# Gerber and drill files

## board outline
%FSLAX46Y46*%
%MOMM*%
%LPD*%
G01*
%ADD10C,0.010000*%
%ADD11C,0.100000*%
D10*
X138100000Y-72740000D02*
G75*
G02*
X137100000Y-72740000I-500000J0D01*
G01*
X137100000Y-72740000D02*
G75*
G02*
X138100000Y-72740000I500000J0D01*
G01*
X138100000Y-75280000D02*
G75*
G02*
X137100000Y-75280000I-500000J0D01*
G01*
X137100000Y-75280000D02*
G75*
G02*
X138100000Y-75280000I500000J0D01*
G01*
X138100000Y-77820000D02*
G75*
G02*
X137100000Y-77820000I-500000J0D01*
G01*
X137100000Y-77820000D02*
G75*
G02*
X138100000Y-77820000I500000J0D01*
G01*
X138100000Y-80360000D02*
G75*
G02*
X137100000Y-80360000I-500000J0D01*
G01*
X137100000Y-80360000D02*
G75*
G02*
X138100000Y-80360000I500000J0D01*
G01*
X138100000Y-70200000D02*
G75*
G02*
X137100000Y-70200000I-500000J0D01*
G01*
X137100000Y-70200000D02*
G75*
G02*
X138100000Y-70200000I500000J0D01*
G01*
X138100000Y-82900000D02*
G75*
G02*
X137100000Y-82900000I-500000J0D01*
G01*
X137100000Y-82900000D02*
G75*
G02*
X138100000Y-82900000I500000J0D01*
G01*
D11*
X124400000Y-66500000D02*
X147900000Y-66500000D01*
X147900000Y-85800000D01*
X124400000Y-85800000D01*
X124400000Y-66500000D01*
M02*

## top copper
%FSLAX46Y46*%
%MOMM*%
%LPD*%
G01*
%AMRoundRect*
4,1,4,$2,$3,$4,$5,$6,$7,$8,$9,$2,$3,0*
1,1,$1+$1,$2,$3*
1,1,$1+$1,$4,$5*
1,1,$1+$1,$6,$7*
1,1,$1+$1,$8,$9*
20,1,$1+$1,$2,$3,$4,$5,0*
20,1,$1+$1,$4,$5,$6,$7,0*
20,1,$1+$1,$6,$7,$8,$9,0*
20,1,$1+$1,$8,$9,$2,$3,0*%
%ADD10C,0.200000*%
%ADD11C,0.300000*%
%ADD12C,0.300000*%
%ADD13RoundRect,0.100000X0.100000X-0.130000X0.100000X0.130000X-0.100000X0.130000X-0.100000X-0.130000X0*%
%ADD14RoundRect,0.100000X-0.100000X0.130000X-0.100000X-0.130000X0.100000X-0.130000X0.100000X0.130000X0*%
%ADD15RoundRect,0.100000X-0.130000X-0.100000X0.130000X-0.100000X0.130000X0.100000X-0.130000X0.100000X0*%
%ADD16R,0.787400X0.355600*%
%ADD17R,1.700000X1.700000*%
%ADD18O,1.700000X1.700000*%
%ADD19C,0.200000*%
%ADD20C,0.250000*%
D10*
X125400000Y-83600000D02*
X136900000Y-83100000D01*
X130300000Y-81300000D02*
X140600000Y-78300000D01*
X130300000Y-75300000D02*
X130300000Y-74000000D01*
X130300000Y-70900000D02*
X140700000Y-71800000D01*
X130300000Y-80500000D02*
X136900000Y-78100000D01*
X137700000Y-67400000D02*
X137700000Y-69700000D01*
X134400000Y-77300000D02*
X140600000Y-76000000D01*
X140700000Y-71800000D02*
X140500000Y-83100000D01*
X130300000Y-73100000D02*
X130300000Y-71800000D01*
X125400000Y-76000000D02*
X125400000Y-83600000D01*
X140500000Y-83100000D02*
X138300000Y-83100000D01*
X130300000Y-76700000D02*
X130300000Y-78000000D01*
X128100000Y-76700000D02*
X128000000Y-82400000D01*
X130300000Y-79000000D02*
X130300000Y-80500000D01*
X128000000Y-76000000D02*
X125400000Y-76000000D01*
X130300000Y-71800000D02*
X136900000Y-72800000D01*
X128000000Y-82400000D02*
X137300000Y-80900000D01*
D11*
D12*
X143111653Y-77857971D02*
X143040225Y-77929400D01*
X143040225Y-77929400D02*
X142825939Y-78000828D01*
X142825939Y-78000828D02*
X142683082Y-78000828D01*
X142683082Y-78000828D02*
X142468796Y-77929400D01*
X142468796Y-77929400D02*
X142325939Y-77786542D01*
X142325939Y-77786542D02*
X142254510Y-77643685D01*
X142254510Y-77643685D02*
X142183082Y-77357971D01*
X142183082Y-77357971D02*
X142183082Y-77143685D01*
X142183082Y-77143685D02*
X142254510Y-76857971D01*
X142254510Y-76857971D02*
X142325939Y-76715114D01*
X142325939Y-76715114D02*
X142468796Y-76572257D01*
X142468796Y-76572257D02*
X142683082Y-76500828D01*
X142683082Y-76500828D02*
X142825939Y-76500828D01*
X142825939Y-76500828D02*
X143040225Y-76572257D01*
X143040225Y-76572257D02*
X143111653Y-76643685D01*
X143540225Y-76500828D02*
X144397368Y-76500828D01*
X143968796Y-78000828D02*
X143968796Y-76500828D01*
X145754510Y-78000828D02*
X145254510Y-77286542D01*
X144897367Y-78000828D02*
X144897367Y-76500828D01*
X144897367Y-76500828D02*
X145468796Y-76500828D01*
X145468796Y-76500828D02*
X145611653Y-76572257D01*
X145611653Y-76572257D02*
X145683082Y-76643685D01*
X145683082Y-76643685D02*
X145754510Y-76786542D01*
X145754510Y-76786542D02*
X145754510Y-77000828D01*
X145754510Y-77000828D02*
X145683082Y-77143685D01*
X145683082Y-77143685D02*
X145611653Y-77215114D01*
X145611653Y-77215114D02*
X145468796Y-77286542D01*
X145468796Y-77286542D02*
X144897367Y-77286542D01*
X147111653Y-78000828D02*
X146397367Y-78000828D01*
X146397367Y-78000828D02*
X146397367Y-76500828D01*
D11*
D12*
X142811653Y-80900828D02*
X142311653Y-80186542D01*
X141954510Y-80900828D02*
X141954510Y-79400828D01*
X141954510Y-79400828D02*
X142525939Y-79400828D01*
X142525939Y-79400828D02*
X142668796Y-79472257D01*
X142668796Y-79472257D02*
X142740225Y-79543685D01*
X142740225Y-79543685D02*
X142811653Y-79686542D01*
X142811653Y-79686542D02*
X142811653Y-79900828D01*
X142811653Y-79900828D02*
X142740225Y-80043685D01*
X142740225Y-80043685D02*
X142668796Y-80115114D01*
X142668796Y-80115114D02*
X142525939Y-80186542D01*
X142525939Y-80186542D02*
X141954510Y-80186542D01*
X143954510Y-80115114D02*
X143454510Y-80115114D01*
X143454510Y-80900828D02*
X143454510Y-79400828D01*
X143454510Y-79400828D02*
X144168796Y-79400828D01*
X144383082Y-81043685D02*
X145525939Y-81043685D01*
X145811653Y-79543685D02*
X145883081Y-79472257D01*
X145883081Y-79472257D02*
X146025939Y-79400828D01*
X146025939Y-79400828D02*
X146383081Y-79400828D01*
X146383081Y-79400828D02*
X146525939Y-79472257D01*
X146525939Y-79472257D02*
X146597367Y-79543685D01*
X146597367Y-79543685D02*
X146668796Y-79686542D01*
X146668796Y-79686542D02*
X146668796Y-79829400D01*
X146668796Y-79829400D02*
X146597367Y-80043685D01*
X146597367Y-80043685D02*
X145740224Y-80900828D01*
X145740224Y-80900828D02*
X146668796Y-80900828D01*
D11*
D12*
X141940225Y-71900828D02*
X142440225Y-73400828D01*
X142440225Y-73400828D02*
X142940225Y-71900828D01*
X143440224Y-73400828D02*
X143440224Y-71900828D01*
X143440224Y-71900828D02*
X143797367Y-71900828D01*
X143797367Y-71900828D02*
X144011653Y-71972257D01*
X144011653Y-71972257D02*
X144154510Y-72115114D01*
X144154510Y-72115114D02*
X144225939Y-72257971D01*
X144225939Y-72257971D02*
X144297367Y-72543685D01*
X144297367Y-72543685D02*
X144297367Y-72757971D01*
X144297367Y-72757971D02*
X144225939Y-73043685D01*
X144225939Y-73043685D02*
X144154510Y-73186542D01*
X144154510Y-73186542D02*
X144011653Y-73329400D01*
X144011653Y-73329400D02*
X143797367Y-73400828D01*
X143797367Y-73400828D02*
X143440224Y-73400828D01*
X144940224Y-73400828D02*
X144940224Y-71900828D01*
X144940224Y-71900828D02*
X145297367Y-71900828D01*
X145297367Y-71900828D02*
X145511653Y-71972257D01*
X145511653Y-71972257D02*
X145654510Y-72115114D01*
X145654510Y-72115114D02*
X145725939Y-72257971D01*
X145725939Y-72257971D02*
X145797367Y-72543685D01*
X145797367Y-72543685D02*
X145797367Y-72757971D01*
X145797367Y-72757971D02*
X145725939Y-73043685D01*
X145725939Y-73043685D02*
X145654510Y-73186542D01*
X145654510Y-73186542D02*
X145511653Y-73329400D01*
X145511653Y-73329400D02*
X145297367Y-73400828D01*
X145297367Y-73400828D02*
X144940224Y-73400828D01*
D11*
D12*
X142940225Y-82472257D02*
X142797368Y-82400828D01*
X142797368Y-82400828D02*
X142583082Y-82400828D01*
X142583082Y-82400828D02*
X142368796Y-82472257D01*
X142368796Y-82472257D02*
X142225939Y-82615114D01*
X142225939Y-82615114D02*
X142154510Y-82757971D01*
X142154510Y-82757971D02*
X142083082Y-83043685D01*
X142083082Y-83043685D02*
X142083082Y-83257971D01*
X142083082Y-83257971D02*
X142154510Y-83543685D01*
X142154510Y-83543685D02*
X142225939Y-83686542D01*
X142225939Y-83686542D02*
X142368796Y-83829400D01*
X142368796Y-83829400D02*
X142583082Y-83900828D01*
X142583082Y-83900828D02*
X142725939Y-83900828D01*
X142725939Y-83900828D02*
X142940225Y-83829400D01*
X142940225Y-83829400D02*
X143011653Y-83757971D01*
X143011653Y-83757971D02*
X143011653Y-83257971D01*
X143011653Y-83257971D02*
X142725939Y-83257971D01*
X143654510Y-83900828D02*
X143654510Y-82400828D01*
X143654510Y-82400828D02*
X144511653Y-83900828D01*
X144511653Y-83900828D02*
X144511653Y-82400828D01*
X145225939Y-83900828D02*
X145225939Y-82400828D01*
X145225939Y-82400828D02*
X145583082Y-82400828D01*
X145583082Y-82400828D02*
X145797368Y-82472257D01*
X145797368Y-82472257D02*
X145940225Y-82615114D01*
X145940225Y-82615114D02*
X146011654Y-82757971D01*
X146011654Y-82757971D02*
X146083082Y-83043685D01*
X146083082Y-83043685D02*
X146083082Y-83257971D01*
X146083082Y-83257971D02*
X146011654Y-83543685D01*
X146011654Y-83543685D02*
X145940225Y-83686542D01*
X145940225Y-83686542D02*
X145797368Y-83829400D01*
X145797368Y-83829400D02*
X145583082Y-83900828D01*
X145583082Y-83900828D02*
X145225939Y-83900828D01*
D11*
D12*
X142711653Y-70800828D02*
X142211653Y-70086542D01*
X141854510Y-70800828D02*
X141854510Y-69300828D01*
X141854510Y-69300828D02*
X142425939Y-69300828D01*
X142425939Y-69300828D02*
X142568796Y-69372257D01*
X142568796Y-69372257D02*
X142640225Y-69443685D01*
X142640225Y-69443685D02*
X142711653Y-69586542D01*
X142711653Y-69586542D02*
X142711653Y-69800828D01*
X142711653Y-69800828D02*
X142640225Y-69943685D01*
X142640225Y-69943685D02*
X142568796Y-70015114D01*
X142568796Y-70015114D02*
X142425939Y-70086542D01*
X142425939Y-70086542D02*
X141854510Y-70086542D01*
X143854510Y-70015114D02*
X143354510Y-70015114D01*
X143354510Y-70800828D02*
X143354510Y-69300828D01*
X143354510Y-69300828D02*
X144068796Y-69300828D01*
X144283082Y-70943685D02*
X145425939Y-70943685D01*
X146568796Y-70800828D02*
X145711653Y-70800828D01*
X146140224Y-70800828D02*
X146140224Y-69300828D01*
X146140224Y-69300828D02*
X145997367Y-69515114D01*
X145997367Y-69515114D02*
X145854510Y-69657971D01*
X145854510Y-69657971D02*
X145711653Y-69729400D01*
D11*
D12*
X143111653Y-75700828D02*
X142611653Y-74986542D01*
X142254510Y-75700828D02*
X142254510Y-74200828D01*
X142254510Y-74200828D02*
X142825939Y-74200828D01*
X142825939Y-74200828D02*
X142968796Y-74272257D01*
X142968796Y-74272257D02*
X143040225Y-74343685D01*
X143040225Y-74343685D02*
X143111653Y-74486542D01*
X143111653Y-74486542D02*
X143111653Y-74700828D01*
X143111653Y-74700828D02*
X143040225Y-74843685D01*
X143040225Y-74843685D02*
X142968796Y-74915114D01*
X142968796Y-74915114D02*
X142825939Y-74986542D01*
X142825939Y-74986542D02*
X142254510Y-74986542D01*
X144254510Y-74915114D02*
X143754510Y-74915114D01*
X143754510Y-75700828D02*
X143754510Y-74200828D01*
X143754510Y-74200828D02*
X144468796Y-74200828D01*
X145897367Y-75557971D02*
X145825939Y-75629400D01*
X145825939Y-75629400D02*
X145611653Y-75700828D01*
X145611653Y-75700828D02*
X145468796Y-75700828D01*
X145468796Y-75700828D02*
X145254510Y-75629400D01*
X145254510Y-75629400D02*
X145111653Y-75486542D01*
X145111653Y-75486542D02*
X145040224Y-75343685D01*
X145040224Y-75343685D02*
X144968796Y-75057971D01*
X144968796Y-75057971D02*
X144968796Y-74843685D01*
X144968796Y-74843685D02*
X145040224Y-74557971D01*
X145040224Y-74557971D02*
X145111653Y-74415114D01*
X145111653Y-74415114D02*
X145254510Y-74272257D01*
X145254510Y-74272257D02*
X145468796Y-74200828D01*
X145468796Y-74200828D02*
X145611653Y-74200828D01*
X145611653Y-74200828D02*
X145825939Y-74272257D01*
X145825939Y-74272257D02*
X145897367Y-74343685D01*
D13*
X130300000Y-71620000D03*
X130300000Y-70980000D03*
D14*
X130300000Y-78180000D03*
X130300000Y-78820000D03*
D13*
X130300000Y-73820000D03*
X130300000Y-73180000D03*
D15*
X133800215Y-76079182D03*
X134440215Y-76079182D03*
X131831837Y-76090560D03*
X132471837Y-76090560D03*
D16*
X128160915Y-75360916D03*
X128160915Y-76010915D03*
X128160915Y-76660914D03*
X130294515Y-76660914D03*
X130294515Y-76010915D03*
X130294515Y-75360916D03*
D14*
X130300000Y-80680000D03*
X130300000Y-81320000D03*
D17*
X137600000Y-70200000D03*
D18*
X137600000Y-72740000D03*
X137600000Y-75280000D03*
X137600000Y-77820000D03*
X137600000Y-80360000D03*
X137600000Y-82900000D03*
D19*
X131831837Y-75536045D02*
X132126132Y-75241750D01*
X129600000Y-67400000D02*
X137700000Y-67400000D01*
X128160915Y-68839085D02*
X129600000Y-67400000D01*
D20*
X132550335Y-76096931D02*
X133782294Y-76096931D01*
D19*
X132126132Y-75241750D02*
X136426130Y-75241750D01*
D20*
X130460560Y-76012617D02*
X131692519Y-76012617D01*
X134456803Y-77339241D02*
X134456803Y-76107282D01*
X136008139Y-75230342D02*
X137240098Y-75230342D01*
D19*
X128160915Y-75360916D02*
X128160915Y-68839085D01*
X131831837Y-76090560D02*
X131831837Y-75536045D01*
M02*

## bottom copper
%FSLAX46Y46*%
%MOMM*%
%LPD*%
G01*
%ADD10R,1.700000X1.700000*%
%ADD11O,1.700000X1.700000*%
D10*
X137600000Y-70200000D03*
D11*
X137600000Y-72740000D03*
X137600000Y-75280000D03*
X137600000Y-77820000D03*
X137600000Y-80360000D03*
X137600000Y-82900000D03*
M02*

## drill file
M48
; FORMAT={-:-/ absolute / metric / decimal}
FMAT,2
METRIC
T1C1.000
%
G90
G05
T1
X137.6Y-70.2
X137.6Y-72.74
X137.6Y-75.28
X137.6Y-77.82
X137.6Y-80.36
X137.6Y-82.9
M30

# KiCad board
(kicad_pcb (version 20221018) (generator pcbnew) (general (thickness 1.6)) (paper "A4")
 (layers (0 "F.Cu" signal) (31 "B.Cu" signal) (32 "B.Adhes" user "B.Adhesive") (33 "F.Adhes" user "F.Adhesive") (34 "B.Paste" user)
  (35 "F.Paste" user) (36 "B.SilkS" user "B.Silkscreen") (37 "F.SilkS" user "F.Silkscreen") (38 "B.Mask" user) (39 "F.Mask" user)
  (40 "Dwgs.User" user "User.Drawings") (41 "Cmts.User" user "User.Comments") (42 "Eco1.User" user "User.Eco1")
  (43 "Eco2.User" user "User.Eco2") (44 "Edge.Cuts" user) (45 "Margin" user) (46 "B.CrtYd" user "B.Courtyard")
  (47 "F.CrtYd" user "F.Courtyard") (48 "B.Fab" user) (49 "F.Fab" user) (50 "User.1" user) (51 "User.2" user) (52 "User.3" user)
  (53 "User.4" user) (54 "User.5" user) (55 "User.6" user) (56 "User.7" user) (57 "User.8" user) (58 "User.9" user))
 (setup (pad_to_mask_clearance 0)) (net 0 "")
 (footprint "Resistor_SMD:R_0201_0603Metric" (layer "F.Cu") (at 130.3 71.3 90)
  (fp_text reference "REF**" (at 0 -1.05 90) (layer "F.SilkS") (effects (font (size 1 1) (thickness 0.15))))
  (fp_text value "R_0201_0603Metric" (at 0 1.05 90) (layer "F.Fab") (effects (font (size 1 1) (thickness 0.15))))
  (pad "" smd roundrect (at -0.345 0 90) (size 0.318 0.36) (layers "F.Paste") (roundrect_rratio 0.25))
  (pad "" smd roundrect (at 0.345 0 90) (size 0.318 0.36) (layers "F.Paste") (roundrect_rratio 0.25))
  (pad "1" smd roundrect (at -0.32 0 90) (size 0.46 0.4) (layers "F.Cu" "F.Mask") (roundrect_rratio 0.25))
  (pad "2" smd roundrect (at 0.32 0 90) (size 0.46 0.4) (layers "F.Cu" "F.Mask") (roundrect_rratio 0.25)))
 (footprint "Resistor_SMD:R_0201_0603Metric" (layer "F.Cu") (at 130.3 78.5 -90)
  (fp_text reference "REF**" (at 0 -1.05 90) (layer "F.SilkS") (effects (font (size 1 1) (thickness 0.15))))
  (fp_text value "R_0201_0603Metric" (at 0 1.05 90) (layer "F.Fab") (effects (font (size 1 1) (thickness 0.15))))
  (pad "" smd roundrect (at -0.345 0 270) (size 0.318 0.36) (layers "F.Paste") (roundrect_rratio 0.25))
  (pad "" smd roundrect (at 0.345 0 270) (size 0.318 0.36) (layers "F.Paste") (roundrect_rratio 0.25))
  (pad "1" smd roundrect (at -0.32 0 270) (size 0.46 0.4) (layers "F.Cu" "F.Mask") (roundrect_rratio 0.25))
  (pad "2" smd roundrect (at 0.32 0 270) (size 0.46 0.4) (layers "F.Cu" "F.Mask") (roundrect_rratio 0.25)))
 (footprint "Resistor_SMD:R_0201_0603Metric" (layer "F.Cu") (at 130.3 73.5 90)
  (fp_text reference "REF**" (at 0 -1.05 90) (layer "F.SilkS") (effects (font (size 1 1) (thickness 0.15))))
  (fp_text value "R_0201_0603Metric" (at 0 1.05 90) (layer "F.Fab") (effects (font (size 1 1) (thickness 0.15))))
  (pad "" smd roundrect (at -0.345 0 90) (size 0.318 0.36) (layers "F.Paste") (roundrect_rratio 0.25))
  (pad "" smd roundrect (at 0.345 0 90) (size 0.318 0.36) (layers "F.Paste") (roundrect_rratio 0.25))
  (pad "1" smd roundrect (at -0.32 0 90) (size 0.46 0.4) (layers "F.Cu" "F.Mask") (roundrect_rratio 0.25))
  (pad "2" smd roundrect (at 0.32 0 90) (size 0.46 0.4) (layers "F.Cu" "F.Mask") (roundrect_rratio 0.25)))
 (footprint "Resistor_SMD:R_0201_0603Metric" (layer "F.Cu") (at 134.120215 76.079182)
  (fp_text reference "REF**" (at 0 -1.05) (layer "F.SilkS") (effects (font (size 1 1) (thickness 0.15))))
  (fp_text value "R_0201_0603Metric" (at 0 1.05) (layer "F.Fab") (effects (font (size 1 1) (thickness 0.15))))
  (pad "" smd roundrect (at -0.345 0) (size 0.318 0.36) (layers "F.Paste") (roundrect_rratio 0.25))
  (pad "" smd roundrect (at 0.345 0) (size 0.318 0.36) (layers "F.Paste") (roundrect_rratio 0.25))
  (pad "1" smd roundrect (at -0.32 0) (size 0.46 0.4) (layers "F.Cu" "F.Mask") (roundrect_rratio 0.25))
  (pad "2" smd roundrect (at 0.32 0) (size 0.46 0.4) (layers "F.Cu" "F.Mask") (roundrect_rratio 0.25)))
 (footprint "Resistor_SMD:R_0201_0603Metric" (layer "F.Cu") (at 132.151837 76.09056)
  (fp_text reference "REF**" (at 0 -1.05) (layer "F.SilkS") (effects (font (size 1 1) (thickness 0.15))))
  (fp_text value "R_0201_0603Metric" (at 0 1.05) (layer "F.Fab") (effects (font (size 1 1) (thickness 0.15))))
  (pad "" smd roundrect (at -0.345 0) (size 0.318 0.36) (layers "F.Paste") (roundrect_rratio 0.25))
  (pad "" smd roundrect (at 0.345 0) (size 0.318 0.36) (layers "F.Paste") (roundrect_rratio 0.25))
  (pad "1" smd roundrect (at -0.32 0) (size 0.46 0.4) (layers "F.Cu" "F.Mask") (roundrect_rratio 0.25))
  (pad "2" smd roundrect (at 0.32 0) (size 0.46 0.4) (layers "F.Cu" "F.Mask") (roundrect_rratio 0.25)))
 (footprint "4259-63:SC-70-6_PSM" (layer "F.Cu") (at 129.227715 76.010915)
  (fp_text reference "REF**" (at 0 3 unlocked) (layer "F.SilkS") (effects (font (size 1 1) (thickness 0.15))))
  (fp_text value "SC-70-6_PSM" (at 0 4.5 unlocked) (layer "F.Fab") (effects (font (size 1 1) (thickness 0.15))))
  (pad "1" smd rect (at -1.0668 -0.649999) (size 0.7874 0.3556) (layers "F.Cu" "F.Paste" "F.Mask"))
  (pad "2" smd rect (at -1.0668 0) (size 0.7874 0.3556) (layers "F.Cu" "F.Paste" "F.Mask"))
  (pad "3" smd rect (at -1.0668 0.649999) (size 0.7874 0.3556) (layers "F.Cu" "F.Paste" "F.Mask"))
  (pad "4" smd rect (at 1.0668 0.649999) (size 0.7874 0.3556) (layers "F.Cu" "F.Paste" "F.Mask"))
  (pad "5" smd rect (at 1.0668 0) (size 0.7874 0.3556) (layers "F.Cu" "F.Paste" "F.Mask"))
  (pad "6" smd rect (at 1.0668 -0.649999) (size 0.7874 0.3556) (layers "F.Cu" "F.Paste" "F.Mask")))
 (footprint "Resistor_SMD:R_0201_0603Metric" (layer "F.Cu") (at 130.3 81 -90)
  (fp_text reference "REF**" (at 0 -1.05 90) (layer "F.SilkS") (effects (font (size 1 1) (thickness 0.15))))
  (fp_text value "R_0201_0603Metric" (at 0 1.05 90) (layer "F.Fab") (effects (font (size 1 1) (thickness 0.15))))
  (pad "" smd roundrect (at -0.345 0 270) (size 0.318 0.36) (layers "F.Paste") (roundrect_rratio 0.25))
  (pad "" smd roundrect (at 0.345 0 270) (size 0.318 0.36) (layers "F.Paste") (roundrect_rratio 0.25))
  (pad "1" smd roundrect (at -0.32 0 270) (size 0.46 0.4) (layers "F.Cu" "F.Mask") (roundrect_rratio 0.25))
  (pad "2" smd roundrect (at 0.32 0 270) (size 0.46 0.4) (layers "F.Cu" "F.Mask") (roundrect_rratio 0.25)))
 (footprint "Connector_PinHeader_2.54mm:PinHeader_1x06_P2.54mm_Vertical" (layer "F.Cu") (at 137.6 70.2)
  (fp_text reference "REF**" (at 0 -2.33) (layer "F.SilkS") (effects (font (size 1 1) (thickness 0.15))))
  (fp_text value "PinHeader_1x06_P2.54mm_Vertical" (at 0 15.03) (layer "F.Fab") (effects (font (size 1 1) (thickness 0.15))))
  (pad "1" thru_hole rect (at 0 0) (size 1.7 1.7) (drill 1) (layers "*.Cu" "*.Mask"))
  (pad "2" thru_hole oval (at 0 2.54) (size 1.7 1.7) (drill 1) (layers "*.Cu" "*.Mask"))
  (pad "3" thru_hole oval (at 0 5.08) (size 1.7 1.7) (drill 1) (layers "*.Cu" "*.Mask"))
  (pad "4" thru_hole oval (at 0 7.62) (size 1.7 1.7) (drill 1) (layers "*.Cu" "*.Mask"))
  (pad "5" thru_hole oval (at 0 10.16) (size 1.7 1.7) (drill 1) (layers "*.Cu" "*.Mask"))
  (pad "6" thru_hole oval (at 0 12.7) (size 1.7 1.7) (drill 1) (layers "*.Cu" "*.Mask")))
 (gr_line (start 125.4 83.6) (end 136.9 83.1) (stroke (width 0.2) (type default)) (layer "F.Cu"))
 (gr_line (start 130.3 81.3) (end 140.6 78.3) (stroke (width 0.2) (type default)) (layer "F.Cu"))
 (gr_line (start 130.3 75.3) (end 130.3 74) (stroke (width 0.2) (type default)) (layer "F.Cu"))
 (gr_line (start 130.3 70.9) (end 140.7 71.8) (stroke (width 0.2) (type default)) (layer "F.Cu"))
 (gr_line (start 130.3 80.5) (end 136.9 78.1) (stroke (width 0.2) (type default)) (layer "F.Cu"))
 (gr_line (start 137.7 67.4) (end 137.7 69.7) (stroke (width 0.2) (type default)) (layer "F.Cu"))
 (gr_line (start 134.4 77.3) (end 140.6 76) (stroke (width 0.2) (type default)) (layer "F.Cu"))
 (gr_line (start 140.7 71.8) (end 140.5 83.1) (stroke (width 0.2) (type default)) (layer "F.Cu"))
 (gr_line (start 130.3 73.1) (end 130.3 71.8) (stroke (width 0.2) (type default)) (layer "F.Cu"))
 (gr_line (start 125.4 76) (end 125.4 83.6) (stroke (width 0.2) (type default)) (layer "F.Cu"))
 (gr_line (start 140.5 83.1) (end 138.3 83.1) (stroke (width 0.2) (type default)) (layer "F.Cu"))
 (gr_line (start 130.3 76.7) (end 130.3 78) (stroke (width 0.2) (type default)) (layer "F.Cu"))
 (gr_line (start 128.1 76.7) (end 128 82.4) (stroke (width 0.2) (type default)) (layer "F.Cu"))
 (gr_line (start 130.3 79) (end 130.3 80.5) (stroke (width 0.2) (type default)) (layer "F.Cu"))
 (gr_line (start 128 76) (end 125.4 76) (stroke (width 0.2) (type default)) (layer "F.Cu"))
 (gr_line (start 130.3 71.8) (end 136.9 72.8) (stroke (width 0.2) (type default)) (layer "F.Cu"))
 (gr_line (start 128 82.4) (end 137.3 80.9) (stroke (width 0.2) (type default)) (layer "F.Cu"))
 (gr_circle (center 137.6 72.74) (end 138.1 72.74) (stroke (width 0.01) (type default)) (fill none) (layer "Edge.Cuts"))
 (gr_circle (center 137.6 75.28) (end 138.1 75.28) (stroke (width 0.01) (type default)) (fill none) (layer "Edge.Cuts"))
 (gr_circle (center 137.6 77.82) (end 138.1 77.82) (stroke (width 0.01) (type default)) (fill none) (layer "Edge.Cuts"))
 (gr_circle (center 137.6 80.36) (end 138.1 80.36) (stroke (width 0.01) (type default)) (fill none) (layer "Edge.Cuts"))
 (gr_circle (center 137.6 70.2) (end 138.1 70.2) (stroke (width 0.01) (type default)) (fill none) (layer "Edge.Cuts"))
 (gr_circle (center 137.6 82.9) (end 138.1 82.9) (stroke (width 0.01) (type default)) (fill none) (layer "Edge.Cuts"))
 (gr_rect (start 124.4 66.5) (end 147.9 85.8) (stroke (width 0.1) (type default)) (fill none) (layer "Edge.Cuts"))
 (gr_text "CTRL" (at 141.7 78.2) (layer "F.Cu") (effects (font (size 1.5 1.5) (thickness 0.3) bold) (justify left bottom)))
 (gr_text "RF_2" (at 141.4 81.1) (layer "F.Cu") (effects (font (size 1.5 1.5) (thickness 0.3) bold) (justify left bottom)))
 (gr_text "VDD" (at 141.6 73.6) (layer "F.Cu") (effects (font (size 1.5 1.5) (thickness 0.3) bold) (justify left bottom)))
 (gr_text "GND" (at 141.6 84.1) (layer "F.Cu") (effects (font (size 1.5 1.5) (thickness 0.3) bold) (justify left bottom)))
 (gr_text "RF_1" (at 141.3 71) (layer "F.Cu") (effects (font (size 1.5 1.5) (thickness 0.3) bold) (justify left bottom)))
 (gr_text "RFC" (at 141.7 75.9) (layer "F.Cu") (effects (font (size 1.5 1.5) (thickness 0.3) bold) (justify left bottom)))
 (segment (start 131.831837 75.536045) (end 132.126132 75.24175) (width 0.2) (layer "F.Cu") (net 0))
 (segment (start 129.6 67.4) (end 137.7 67.4) (width 0.2) (layer "F.Cu") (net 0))
 (segment (start 128.160915 68.839085) (end 129.6 67.4) (width 0.2) (layer "F.Cu") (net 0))
 (segment (start 132.550335 76.096931) (end 133.782294 76.096931) (width 0.25) (layer "F.Cu") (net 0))
 (segment (start 132.126132 75.24175) (end 136.42613 75.24175) (width 0.2) (layer "F.Cu") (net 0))
 (segment (start 130.46056 76.012617) (end 131.692519 76.012617) (width 0.25) (layer "F.Cu") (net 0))
 (segment (start 134.456803 77.339241) (end 134.456803 76.107282) (width 0.25) (layer "F.Cu") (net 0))
 (segment (start 136.008139 75.230342) (end 137.240098 75.230342) (width 0.25) (layer "F.Cu") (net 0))
 (segment (start 128.160915 75.360916) (end 128.160915 68.839085) (width 0.2) (layer "F.Cu") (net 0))
 (segment (start 131.831837 76.09056) (end 131.831837 75.536045) (width 0.2) (layer "F.Cu") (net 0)))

